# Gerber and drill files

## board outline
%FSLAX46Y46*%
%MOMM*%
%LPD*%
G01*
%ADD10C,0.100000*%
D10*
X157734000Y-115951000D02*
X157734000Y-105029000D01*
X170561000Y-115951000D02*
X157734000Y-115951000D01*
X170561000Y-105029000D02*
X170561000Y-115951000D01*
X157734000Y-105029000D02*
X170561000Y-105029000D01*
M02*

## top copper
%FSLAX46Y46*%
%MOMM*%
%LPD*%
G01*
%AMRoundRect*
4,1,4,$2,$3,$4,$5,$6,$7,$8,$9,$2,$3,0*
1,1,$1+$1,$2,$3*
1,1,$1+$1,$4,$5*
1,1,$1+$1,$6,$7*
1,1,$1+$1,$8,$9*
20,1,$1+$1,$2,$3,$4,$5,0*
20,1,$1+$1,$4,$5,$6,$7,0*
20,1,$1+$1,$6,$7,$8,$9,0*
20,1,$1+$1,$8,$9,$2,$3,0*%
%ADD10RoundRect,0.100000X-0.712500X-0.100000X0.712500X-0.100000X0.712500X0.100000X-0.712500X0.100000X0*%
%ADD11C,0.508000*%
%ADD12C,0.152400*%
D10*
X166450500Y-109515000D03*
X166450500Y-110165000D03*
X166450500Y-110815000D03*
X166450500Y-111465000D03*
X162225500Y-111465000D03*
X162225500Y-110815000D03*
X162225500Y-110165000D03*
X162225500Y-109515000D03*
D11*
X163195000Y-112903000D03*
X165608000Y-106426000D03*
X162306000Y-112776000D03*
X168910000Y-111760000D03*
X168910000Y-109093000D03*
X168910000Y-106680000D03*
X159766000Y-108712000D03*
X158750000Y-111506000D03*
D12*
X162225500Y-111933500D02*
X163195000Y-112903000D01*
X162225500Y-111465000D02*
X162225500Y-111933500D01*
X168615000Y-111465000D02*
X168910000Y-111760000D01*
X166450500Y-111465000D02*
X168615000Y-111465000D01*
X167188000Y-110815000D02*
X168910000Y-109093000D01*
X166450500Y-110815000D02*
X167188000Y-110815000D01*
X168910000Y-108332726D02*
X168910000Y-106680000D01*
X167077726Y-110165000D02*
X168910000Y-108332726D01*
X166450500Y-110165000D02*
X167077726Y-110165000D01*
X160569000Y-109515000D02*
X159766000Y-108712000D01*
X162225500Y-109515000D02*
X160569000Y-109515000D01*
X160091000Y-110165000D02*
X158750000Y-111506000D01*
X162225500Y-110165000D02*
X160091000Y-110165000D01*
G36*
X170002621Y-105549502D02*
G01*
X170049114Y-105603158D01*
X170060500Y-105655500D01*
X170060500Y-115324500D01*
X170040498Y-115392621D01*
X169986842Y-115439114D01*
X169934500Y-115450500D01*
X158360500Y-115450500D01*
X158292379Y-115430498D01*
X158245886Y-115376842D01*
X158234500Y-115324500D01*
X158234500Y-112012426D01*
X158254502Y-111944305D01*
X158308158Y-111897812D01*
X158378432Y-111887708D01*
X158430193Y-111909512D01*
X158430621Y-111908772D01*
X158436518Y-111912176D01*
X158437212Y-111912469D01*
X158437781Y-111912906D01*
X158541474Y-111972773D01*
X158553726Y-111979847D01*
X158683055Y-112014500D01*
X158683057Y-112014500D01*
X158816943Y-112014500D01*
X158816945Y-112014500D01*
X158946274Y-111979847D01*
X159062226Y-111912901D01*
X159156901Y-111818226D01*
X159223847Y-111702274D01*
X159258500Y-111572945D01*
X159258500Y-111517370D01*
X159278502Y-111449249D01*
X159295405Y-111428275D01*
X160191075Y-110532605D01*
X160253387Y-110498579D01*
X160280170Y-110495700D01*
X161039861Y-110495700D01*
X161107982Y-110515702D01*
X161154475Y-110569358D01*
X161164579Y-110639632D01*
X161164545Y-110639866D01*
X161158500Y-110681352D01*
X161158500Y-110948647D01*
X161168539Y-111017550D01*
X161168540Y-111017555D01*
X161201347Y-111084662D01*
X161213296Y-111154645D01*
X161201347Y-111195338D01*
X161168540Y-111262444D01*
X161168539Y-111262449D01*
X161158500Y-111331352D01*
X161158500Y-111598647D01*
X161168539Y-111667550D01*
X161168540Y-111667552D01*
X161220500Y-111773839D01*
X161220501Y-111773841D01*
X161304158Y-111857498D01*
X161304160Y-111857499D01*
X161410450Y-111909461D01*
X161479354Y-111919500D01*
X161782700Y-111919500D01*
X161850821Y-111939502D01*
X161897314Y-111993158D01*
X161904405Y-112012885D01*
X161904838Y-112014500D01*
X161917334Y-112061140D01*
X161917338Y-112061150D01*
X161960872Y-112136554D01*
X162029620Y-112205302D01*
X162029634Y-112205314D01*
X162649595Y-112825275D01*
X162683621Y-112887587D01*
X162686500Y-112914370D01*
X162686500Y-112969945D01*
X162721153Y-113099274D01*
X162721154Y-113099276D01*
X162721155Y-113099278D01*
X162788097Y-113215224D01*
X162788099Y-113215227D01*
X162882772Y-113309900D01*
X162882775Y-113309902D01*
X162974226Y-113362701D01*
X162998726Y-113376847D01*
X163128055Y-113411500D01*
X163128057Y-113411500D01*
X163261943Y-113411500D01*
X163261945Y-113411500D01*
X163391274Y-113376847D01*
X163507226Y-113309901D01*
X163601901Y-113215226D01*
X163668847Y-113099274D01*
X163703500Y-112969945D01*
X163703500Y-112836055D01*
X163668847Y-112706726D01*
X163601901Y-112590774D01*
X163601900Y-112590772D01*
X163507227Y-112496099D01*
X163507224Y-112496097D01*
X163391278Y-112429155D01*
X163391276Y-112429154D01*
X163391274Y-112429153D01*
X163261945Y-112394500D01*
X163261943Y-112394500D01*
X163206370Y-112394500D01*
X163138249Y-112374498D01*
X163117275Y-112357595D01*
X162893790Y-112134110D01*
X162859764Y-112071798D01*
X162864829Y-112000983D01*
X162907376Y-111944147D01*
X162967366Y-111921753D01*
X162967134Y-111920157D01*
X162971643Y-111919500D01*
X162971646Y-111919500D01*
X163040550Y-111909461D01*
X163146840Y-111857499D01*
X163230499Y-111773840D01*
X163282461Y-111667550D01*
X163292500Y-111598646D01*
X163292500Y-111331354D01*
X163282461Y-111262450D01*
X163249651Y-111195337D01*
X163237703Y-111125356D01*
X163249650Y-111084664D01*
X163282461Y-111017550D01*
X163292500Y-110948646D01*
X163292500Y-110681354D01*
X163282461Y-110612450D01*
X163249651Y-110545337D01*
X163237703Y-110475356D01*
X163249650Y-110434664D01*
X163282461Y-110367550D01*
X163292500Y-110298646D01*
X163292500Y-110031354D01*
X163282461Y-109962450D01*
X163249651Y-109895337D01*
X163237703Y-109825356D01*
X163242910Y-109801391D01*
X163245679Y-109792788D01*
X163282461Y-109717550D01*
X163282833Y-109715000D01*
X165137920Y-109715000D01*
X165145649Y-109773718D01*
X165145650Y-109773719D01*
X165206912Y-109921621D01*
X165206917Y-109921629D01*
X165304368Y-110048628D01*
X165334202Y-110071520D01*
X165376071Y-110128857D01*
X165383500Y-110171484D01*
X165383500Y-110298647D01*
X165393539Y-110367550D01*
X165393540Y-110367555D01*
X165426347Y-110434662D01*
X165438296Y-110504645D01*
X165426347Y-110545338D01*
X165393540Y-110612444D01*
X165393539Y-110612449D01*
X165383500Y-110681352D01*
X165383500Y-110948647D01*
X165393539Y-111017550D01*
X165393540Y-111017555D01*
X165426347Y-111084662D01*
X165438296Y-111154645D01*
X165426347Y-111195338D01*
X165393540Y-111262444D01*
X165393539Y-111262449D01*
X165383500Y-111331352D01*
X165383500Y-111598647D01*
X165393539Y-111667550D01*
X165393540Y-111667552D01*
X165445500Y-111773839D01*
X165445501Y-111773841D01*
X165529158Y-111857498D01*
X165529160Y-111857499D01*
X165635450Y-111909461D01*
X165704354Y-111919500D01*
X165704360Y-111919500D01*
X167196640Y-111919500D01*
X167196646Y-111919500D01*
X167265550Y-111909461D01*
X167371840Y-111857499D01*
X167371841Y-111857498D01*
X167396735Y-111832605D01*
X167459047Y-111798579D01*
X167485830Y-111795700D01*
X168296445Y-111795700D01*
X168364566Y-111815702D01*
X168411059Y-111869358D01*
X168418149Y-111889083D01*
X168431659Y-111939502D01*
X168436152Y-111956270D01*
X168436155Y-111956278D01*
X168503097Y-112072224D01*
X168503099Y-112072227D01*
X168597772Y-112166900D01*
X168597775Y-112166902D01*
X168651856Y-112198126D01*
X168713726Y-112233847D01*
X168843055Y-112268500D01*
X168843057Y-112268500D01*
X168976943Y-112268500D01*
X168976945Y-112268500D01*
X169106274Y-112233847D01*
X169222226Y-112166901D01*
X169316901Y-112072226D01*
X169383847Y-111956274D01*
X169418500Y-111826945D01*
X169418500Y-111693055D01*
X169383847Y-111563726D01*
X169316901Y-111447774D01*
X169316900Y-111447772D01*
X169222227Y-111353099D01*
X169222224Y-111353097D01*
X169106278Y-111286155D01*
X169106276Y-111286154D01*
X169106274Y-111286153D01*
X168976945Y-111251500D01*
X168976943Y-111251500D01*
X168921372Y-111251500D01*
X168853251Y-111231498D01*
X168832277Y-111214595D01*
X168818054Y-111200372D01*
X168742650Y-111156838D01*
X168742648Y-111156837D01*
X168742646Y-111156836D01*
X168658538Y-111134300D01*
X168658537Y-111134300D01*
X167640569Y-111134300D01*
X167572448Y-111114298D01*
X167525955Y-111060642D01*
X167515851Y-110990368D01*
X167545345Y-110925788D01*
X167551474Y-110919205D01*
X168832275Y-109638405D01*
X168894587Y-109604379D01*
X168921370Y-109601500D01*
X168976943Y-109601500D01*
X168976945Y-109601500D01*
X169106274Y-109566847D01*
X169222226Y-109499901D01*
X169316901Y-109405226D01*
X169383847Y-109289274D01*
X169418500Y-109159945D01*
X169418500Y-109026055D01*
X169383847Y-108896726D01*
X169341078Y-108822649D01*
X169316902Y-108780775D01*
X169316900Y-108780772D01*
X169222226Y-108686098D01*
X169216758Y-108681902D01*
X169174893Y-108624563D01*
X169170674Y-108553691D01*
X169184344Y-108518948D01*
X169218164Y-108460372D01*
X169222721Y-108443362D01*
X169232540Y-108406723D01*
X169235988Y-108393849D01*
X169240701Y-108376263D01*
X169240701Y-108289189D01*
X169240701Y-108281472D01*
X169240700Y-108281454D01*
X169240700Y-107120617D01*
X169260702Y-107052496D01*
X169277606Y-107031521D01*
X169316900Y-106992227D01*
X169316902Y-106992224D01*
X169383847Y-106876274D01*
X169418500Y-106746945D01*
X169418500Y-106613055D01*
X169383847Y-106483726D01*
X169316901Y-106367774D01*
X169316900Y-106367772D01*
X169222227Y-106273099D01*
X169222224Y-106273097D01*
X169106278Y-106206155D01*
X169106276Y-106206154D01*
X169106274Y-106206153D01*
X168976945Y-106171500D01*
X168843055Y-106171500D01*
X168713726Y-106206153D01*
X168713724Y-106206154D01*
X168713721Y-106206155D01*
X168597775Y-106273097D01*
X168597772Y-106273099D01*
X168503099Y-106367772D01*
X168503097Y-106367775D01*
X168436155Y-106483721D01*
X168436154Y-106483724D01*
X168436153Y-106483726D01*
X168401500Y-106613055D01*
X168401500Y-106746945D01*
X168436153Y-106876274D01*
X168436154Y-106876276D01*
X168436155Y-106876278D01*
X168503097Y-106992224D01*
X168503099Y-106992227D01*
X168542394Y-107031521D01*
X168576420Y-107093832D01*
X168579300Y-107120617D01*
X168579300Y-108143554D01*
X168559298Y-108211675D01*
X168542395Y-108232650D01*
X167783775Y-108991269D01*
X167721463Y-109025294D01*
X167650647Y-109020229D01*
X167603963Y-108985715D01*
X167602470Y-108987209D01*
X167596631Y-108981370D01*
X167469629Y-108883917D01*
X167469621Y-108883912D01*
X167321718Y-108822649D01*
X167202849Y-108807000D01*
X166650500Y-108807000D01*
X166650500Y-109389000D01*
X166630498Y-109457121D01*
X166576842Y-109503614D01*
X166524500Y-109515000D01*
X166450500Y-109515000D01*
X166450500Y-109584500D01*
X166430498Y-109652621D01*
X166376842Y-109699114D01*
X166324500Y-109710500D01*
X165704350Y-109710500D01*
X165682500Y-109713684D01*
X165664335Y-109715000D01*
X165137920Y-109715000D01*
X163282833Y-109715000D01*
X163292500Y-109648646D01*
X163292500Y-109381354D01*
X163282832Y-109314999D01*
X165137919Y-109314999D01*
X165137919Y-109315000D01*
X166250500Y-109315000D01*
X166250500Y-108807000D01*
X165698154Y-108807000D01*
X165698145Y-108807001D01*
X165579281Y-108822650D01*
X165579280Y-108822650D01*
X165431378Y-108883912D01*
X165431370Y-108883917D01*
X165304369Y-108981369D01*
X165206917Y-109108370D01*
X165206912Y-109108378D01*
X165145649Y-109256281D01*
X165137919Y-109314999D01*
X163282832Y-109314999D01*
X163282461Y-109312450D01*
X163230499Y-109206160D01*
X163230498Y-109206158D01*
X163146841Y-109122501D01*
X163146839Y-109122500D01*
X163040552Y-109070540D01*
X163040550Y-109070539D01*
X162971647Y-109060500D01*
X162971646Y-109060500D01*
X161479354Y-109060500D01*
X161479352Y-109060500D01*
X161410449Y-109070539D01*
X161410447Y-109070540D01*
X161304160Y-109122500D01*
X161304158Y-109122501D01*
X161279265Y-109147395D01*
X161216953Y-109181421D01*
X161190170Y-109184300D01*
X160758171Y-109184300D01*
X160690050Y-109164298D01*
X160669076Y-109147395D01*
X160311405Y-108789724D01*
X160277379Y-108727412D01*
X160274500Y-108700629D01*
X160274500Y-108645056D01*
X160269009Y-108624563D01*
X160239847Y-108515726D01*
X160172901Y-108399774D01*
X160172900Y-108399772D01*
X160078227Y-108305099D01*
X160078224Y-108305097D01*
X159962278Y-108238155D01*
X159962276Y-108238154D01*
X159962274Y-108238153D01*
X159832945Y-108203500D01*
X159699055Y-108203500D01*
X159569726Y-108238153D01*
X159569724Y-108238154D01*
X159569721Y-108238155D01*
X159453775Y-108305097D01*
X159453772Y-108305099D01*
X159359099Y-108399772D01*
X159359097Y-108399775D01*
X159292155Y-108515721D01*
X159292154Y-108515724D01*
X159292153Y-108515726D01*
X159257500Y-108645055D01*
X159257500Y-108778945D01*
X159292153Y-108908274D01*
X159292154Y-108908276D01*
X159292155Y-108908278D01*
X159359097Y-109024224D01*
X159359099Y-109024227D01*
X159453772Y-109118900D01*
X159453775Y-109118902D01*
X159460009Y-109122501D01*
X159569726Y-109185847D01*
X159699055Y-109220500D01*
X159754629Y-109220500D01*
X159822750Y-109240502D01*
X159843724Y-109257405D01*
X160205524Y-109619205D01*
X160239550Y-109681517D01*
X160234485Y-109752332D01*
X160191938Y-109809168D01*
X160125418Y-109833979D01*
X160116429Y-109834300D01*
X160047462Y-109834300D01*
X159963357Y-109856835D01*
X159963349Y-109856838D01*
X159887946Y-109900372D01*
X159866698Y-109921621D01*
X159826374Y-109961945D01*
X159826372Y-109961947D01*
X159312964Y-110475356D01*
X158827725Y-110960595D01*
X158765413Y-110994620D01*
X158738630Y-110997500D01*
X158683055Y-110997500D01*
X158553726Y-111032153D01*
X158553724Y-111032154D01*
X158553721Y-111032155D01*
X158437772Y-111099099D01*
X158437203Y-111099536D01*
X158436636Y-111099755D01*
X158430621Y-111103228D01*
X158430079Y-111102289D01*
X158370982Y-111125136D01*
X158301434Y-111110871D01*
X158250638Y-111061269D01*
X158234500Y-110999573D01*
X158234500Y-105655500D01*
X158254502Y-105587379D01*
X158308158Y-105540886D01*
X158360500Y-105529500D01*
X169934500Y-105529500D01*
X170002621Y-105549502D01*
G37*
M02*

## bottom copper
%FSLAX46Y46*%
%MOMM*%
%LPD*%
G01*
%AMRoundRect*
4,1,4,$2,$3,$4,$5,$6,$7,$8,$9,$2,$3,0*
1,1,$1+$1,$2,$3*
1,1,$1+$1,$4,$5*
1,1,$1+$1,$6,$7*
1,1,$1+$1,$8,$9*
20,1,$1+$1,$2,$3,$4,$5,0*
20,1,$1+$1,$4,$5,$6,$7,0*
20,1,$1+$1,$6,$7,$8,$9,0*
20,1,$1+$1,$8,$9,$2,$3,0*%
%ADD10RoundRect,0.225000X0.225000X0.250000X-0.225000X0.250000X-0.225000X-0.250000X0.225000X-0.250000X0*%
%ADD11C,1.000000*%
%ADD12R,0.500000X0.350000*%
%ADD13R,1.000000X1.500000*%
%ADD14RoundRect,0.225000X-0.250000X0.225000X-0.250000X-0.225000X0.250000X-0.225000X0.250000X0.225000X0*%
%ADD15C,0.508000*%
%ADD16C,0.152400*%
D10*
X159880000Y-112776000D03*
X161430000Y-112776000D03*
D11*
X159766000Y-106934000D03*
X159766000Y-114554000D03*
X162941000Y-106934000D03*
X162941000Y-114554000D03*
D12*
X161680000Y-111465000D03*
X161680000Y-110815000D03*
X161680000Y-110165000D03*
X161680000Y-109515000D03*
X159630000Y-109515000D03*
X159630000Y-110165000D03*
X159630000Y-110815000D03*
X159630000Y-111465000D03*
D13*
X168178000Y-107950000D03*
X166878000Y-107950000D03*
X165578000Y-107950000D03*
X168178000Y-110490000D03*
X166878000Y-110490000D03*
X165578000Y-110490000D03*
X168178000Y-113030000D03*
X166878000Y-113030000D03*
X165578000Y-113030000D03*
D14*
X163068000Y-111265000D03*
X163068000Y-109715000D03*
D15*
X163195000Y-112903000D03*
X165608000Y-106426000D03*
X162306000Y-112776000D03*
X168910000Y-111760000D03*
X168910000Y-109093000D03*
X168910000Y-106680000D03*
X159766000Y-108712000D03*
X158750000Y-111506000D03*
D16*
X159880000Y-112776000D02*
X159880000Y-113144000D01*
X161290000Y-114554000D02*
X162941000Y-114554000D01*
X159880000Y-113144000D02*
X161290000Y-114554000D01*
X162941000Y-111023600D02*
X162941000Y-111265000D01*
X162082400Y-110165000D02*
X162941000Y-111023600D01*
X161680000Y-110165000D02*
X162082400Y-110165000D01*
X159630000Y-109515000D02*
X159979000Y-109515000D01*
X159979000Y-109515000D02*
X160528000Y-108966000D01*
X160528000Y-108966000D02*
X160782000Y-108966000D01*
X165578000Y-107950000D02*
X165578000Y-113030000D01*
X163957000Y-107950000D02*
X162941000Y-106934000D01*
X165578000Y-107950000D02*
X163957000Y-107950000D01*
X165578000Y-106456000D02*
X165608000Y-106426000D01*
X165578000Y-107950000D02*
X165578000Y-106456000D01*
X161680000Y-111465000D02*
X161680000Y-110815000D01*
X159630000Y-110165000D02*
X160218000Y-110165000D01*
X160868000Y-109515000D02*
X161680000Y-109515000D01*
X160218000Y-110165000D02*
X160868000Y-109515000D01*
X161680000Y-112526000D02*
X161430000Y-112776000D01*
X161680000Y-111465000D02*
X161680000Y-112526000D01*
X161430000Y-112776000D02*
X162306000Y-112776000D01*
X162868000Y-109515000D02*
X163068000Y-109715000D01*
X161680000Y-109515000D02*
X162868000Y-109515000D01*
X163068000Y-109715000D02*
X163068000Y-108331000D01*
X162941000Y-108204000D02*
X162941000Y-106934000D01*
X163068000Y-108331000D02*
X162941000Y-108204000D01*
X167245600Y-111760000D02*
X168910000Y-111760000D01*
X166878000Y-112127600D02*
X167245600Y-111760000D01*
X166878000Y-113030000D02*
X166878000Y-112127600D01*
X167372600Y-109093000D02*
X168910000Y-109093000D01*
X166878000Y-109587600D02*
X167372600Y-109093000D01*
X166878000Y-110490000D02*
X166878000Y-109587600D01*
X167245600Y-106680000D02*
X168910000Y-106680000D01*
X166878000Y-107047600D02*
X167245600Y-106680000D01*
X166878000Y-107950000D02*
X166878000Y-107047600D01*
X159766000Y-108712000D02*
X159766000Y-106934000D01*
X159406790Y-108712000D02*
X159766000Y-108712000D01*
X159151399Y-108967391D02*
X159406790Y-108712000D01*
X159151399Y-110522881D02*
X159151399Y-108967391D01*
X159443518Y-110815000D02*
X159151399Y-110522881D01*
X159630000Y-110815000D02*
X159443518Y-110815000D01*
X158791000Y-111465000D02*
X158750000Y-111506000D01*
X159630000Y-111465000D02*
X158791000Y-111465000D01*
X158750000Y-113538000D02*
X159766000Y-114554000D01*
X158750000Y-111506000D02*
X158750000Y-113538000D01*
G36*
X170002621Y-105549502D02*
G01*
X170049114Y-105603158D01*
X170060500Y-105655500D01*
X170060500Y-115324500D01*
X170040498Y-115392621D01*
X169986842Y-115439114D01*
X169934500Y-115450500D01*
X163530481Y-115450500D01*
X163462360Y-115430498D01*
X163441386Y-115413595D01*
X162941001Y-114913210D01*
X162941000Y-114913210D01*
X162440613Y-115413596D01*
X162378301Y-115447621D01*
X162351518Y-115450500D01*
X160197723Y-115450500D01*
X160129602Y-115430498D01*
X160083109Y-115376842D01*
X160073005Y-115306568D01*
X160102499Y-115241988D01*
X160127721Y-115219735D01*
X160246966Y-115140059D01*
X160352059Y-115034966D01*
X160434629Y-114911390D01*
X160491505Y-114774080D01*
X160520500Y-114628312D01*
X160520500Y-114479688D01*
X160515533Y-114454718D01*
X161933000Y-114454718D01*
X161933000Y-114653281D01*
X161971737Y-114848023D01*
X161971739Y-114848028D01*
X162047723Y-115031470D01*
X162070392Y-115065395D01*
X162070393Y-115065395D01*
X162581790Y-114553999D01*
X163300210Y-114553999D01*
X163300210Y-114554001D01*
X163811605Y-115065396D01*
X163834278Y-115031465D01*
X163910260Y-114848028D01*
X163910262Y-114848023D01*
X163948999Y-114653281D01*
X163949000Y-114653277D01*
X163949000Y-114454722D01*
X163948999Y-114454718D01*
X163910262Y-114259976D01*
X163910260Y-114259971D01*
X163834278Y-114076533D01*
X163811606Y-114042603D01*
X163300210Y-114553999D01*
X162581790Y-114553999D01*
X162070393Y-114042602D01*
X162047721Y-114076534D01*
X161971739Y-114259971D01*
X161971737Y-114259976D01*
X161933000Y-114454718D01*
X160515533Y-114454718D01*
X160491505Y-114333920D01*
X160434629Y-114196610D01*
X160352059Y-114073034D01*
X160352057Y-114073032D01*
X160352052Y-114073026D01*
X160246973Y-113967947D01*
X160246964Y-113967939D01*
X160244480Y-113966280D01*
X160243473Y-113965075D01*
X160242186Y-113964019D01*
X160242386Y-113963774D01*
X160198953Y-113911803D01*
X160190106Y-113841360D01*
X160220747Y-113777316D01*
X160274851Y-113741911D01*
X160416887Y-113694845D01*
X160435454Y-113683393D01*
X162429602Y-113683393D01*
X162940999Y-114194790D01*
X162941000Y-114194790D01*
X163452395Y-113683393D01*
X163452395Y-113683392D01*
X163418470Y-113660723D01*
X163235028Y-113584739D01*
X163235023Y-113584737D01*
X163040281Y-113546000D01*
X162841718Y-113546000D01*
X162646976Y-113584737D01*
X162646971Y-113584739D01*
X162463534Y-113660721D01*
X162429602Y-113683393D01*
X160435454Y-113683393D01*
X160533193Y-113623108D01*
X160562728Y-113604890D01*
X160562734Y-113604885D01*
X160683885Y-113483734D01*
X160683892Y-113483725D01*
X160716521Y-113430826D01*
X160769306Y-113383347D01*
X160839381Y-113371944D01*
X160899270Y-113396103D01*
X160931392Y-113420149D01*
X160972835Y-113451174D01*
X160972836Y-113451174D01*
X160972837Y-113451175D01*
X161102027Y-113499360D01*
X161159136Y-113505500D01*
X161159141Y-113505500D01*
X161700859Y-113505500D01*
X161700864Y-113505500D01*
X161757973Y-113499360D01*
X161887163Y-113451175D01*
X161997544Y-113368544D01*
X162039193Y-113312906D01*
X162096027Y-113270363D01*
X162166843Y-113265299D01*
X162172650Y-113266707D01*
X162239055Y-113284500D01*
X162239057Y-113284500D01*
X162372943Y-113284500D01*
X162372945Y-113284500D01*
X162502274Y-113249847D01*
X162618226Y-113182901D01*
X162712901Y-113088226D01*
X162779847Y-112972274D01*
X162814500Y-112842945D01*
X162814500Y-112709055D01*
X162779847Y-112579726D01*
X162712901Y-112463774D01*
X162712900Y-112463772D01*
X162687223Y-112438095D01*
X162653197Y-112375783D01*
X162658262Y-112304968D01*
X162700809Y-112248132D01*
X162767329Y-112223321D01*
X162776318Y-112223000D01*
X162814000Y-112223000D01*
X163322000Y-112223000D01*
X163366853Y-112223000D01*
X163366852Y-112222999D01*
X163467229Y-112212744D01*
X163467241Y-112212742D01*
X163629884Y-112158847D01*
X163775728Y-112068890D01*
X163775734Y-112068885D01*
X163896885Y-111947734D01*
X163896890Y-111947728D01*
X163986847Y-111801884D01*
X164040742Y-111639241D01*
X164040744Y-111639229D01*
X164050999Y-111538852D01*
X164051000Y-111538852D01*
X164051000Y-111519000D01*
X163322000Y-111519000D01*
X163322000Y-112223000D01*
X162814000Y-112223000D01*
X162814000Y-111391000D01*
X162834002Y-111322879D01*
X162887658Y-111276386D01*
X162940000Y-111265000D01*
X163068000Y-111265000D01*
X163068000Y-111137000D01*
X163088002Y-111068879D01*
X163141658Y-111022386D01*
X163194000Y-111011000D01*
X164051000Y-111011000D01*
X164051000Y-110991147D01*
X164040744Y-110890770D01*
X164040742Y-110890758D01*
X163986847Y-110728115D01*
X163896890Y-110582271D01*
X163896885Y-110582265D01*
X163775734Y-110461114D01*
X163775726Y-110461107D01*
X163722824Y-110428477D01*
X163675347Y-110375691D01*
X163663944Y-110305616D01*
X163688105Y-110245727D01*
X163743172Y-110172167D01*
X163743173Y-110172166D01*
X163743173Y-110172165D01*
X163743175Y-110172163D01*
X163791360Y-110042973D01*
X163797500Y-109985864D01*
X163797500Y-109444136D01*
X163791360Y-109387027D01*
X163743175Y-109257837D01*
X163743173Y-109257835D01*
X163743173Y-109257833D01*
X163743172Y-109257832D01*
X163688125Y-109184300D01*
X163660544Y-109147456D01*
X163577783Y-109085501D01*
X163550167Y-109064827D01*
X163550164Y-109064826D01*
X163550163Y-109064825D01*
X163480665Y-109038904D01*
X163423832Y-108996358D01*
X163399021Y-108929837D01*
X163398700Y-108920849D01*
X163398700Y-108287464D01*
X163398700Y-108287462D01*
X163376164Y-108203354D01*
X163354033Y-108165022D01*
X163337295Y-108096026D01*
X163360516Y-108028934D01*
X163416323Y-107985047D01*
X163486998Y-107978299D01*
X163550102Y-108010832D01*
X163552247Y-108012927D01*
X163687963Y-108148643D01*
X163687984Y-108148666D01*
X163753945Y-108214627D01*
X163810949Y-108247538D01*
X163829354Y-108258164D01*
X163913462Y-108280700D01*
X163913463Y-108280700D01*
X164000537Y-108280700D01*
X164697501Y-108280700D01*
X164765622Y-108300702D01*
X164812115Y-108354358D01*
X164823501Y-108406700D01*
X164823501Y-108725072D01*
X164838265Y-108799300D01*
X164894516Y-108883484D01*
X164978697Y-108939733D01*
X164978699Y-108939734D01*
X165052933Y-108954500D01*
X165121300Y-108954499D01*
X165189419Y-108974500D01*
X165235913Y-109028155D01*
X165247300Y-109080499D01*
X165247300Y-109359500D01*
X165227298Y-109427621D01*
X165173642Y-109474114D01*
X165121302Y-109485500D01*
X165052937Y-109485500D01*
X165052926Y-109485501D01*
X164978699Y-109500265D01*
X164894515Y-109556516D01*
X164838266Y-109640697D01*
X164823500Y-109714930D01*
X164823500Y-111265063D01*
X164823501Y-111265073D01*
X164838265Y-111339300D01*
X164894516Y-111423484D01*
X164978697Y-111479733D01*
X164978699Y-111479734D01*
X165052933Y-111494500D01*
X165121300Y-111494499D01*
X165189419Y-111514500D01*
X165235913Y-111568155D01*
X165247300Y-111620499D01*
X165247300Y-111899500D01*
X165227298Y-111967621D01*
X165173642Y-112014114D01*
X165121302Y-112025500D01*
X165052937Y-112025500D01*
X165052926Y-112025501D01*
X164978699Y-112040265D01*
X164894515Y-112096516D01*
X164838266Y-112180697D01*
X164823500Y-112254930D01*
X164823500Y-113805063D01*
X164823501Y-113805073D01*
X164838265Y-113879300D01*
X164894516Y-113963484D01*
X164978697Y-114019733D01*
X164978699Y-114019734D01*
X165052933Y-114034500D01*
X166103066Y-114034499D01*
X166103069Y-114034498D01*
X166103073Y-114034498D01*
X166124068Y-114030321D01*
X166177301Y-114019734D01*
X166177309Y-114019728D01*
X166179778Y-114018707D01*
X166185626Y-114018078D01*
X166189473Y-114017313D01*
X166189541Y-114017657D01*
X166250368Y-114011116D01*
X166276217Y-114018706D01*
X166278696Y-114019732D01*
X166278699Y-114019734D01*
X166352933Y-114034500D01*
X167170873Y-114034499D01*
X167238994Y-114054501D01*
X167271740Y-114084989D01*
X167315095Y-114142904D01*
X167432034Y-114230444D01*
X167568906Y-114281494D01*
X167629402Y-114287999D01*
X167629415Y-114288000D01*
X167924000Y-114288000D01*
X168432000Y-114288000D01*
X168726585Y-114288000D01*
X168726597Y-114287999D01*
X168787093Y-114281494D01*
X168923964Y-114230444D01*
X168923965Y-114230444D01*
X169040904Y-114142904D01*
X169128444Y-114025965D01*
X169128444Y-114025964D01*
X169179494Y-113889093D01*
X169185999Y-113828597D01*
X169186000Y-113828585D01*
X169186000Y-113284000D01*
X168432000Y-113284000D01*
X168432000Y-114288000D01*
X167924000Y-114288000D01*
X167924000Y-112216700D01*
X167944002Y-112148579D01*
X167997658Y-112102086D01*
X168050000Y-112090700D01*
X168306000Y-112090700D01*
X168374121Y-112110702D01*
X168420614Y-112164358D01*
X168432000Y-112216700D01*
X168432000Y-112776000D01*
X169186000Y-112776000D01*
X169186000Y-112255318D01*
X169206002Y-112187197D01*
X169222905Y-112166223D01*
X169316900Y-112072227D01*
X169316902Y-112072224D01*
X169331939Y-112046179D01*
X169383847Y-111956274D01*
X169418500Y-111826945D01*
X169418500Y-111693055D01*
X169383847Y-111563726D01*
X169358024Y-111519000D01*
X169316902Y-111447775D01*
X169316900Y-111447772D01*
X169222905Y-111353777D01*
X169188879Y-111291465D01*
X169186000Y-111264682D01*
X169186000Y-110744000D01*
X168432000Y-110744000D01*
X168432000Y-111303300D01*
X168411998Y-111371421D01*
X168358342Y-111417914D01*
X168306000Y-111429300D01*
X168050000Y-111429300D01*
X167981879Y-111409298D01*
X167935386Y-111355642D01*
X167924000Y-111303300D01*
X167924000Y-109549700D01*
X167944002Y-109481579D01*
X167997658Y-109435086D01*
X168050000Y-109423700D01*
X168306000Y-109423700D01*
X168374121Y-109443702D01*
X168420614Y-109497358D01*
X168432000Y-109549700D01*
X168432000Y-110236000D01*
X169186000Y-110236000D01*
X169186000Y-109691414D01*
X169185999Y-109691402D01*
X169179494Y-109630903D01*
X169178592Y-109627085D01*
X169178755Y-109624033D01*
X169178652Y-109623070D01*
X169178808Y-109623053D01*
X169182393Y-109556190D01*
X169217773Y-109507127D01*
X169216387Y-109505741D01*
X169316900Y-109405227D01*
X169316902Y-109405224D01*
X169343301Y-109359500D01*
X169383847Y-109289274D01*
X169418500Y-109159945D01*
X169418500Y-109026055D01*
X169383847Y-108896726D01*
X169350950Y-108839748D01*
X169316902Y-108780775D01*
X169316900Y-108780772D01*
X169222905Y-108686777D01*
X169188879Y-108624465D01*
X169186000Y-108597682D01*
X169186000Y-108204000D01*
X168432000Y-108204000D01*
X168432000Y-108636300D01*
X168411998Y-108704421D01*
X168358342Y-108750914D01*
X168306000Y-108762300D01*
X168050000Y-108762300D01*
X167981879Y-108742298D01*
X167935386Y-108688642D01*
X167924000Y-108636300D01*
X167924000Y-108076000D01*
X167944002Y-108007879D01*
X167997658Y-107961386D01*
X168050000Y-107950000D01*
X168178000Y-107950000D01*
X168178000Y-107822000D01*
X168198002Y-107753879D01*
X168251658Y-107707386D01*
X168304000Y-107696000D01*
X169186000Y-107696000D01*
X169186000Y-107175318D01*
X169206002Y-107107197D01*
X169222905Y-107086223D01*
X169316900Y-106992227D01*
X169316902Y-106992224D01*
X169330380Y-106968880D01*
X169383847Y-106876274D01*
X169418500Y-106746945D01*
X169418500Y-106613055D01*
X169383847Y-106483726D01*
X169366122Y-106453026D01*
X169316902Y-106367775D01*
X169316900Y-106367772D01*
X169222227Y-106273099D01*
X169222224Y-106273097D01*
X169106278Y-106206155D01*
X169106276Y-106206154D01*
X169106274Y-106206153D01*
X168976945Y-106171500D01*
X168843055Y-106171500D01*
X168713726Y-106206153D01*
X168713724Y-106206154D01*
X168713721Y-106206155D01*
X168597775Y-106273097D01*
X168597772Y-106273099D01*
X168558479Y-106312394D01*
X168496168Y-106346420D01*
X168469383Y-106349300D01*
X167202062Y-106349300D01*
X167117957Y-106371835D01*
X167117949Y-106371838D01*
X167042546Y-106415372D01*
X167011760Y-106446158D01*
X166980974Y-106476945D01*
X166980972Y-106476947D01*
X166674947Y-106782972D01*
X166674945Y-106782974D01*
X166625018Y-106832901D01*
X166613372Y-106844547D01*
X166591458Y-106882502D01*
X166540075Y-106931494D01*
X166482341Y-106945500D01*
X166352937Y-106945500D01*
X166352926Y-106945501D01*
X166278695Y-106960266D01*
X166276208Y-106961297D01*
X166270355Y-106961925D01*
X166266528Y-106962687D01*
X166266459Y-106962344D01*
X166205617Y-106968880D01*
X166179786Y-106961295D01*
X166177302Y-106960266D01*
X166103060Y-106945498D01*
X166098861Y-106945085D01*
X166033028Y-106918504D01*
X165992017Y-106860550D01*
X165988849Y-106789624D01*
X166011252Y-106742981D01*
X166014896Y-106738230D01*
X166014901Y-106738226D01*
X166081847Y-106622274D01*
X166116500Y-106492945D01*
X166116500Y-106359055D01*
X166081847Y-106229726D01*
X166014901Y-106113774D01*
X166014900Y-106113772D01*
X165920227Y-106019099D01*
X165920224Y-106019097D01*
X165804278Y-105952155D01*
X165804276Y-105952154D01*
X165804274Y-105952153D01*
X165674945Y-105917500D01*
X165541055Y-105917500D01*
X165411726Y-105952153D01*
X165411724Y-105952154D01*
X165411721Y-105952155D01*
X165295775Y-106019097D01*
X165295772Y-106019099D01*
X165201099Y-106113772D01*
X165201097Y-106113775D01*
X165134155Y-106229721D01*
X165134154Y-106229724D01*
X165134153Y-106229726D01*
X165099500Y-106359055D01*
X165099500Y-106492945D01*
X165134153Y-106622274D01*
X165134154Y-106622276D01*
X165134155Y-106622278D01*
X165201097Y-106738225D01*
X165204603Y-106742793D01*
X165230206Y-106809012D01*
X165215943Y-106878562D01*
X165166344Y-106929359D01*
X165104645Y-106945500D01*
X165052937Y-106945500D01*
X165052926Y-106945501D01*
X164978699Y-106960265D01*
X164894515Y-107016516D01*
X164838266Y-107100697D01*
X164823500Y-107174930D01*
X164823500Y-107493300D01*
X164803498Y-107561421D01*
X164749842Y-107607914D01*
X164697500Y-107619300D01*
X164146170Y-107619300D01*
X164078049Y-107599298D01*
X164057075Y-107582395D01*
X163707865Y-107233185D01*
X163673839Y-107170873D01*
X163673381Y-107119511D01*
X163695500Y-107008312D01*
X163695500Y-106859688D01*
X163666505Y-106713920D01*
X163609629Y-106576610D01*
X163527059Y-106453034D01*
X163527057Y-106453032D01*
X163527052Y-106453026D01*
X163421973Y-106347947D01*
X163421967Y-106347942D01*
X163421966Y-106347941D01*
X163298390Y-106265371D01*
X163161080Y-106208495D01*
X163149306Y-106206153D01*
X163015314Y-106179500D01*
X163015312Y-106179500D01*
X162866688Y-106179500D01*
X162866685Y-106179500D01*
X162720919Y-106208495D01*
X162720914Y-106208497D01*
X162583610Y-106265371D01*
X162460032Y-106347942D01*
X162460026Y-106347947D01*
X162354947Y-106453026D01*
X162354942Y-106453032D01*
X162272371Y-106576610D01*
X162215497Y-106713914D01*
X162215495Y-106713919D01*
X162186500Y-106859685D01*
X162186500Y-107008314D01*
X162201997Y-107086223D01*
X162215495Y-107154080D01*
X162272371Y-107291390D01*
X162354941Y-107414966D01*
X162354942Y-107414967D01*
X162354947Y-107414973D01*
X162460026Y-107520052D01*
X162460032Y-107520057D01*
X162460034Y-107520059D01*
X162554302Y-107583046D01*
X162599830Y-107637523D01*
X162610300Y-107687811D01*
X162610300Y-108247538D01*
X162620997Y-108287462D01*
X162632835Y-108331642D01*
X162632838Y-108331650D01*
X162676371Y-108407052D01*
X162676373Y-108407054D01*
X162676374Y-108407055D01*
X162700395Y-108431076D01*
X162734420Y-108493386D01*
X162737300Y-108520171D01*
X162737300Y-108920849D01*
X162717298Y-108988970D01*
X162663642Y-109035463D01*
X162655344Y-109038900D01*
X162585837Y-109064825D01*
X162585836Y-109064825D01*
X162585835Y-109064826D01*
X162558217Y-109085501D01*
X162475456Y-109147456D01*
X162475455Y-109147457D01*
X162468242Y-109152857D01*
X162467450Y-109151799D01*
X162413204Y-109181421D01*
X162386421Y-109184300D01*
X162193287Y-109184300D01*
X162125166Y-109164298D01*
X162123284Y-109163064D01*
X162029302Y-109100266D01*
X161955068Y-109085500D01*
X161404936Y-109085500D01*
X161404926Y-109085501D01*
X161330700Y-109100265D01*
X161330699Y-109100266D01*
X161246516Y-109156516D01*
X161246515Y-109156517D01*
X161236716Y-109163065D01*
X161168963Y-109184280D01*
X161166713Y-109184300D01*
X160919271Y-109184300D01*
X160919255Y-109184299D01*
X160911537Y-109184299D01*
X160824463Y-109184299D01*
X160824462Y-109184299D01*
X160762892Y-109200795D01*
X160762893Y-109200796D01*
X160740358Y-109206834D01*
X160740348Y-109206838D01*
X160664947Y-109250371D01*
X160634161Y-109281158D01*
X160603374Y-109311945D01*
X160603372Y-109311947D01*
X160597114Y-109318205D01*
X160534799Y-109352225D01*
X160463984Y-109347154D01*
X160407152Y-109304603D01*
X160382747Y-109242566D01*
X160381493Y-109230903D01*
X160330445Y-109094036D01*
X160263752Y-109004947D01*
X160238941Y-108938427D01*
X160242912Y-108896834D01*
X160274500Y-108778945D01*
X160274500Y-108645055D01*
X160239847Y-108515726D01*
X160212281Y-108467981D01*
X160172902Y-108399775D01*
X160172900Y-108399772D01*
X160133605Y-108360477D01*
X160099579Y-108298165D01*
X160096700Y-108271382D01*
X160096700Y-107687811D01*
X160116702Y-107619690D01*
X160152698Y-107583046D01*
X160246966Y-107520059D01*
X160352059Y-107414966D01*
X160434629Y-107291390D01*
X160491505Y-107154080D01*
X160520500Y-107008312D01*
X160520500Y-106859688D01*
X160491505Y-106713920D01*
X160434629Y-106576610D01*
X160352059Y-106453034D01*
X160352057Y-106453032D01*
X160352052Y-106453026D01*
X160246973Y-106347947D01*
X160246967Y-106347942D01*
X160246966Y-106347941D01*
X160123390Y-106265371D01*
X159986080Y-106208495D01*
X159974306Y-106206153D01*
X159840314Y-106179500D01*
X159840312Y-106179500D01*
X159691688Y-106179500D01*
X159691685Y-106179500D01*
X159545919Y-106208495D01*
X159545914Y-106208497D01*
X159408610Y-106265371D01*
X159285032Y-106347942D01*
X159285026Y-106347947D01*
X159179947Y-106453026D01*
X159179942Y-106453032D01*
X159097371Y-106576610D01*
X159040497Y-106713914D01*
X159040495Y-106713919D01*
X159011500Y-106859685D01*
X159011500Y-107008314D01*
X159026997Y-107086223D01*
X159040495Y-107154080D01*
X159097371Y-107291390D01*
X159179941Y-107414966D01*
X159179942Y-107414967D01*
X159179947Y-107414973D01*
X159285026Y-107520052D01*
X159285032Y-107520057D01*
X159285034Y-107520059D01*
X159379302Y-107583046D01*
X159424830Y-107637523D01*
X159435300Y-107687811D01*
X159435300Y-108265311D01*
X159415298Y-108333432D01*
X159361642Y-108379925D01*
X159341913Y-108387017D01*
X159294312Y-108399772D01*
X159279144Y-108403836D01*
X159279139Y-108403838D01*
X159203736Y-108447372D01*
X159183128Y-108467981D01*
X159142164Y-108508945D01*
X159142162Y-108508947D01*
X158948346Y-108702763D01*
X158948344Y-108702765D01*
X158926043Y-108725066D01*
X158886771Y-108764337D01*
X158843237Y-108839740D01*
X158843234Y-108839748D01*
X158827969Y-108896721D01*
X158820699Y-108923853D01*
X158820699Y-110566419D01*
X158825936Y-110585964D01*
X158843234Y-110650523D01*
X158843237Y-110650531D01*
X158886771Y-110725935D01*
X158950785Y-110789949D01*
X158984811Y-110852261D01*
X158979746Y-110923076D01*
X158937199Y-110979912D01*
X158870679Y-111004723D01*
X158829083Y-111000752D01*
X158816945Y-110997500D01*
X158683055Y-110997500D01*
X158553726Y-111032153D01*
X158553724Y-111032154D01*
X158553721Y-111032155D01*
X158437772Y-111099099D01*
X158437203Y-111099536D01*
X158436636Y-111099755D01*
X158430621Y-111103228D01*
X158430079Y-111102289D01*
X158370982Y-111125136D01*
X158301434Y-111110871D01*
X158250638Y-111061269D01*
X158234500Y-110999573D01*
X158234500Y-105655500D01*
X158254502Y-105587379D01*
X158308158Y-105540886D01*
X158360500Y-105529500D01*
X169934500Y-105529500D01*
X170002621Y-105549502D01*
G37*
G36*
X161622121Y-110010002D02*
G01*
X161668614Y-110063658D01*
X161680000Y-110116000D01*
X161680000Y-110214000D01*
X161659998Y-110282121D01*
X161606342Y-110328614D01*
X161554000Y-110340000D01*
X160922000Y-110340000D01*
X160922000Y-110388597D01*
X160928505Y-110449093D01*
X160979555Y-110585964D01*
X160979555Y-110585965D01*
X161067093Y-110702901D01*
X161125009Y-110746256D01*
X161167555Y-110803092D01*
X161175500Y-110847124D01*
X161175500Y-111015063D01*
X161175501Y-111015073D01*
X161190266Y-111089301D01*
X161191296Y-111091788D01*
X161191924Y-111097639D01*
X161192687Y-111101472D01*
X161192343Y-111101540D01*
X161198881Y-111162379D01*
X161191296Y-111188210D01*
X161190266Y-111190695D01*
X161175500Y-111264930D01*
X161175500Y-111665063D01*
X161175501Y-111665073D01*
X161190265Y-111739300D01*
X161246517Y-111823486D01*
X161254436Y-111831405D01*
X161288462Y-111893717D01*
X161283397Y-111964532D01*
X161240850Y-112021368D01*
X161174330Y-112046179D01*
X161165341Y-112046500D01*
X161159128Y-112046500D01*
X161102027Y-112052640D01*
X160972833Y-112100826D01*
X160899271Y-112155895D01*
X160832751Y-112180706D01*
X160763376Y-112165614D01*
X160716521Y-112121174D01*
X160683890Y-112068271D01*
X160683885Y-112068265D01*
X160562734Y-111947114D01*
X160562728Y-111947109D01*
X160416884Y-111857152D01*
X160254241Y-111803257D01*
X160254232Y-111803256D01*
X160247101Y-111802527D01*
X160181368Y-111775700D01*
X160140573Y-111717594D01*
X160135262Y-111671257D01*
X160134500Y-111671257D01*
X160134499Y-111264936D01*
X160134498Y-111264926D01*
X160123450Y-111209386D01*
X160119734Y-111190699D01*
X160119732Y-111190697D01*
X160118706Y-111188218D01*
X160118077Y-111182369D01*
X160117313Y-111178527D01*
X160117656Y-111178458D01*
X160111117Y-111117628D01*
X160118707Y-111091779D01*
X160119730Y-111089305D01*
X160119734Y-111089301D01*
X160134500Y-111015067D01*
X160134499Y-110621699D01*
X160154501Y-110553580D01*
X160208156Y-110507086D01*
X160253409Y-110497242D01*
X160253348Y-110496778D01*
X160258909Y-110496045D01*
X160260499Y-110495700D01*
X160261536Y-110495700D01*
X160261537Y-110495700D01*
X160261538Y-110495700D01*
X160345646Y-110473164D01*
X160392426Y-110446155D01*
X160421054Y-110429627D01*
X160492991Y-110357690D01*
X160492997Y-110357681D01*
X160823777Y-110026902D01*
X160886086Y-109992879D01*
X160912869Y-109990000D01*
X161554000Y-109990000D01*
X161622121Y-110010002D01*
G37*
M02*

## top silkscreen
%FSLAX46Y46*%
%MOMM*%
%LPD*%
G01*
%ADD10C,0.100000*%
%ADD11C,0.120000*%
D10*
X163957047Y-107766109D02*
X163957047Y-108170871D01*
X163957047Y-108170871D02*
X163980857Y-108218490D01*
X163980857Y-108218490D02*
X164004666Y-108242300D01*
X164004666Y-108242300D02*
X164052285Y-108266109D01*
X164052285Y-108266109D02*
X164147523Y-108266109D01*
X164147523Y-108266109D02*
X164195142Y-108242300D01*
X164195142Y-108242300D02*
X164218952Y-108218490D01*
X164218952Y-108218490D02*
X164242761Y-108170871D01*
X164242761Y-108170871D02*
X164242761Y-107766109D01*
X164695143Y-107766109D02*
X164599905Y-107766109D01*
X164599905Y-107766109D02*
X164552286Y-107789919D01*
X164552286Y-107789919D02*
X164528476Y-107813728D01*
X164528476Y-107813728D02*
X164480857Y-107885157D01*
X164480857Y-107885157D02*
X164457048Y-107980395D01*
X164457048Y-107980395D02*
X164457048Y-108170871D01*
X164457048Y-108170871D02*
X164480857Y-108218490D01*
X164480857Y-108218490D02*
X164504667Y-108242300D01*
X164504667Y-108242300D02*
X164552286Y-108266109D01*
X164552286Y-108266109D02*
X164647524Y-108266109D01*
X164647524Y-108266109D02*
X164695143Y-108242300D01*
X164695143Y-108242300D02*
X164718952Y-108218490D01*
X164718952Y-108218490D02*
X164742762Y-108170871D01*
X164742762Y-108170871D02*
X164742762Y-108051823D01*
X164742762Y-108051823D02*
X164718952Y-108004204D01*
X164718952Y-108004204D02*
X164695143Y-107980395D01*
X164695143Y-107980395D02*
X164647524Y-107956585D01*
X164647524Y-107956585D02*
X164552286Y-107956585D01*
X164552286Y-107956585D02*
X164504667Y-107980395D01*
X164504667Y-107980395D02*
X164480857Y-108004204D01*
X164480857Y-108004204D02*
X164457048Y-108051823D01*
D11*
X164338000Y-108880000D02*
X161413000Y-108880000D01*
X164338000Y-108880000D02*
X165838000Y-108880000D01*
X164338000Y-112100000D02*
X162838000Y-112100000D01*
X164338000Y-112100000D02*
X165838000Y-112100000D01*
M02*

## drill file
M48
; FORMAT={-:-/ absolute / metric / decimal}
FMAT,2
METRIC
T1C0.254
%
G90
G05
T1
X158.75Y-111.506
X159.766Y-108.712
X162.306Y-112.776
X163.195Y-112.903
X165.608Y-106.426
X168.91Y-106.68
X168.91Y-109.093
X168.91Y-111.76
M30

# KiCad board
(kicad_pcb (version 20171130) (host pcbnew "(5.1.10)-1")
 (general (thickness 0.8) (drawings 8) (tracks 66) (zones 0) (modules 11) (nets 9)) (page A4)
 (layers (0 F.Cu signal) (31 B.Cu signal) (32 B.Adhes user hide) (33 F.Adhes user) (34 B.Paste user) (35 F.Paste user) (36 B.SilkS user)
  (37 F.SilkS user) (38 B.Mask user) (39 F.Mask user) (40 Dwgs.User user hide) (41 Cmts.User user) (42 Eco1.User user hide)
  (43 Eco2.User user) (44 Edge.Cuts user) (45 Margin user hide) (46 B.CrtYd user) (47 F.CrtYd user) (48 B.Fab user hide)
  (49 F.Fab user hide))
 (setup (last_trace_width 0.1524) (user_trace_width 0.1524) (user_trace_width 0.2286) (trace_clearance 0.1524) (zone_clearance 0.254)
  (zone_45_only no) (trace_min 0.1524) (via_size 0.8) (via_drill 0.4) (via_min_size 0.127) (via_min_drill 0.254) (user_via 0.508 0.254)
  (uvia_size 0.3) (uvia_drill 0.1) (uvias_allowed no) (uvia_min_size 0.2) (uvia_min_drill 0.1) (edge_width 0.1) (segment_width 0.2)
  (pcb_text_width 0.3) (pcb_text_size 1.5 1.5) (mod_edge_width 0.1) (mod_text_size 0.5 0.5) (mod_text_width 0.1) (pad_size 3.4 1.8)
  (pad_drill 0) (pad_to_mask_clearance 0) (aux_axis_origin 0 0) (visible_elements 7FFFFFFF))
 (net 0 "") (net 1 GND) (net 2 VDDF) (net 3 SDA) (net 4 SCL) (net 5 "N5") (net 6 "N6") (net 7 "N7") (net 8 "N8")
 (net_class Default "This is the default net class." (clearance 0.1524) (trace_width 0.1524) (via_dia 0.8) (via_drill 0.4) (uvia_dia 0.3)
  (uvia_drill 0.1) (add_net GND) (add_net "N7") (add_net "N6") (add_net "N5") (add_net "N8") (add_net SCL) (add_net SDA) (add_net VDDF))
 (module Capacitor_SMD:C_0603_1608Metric (layer B.Cu) (at 160.655 112.776 180)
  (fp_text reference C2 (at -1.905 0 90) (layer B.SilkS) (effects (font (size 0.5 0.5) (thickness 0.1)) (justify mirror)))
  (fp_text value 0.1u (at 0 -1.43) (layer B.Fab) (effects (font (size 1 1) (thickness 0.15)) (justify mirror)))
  (pad 2 smd roundrect (at 0.775 0 180) (size 0.9 0.95) (layers B.Cu B.Paste B.Mask) (roundrect_rratio 0.25) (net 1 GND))
  (pad 1 smd roundrect (at -0.775 0 180) (size 0.9 0.95) (layers B.Cu B.Paste B.Mask) (roundrect_rratio 0.25) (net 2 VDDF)))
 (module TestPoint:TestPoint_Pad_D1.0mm (layer B.Cu) (at 159.766 106.934)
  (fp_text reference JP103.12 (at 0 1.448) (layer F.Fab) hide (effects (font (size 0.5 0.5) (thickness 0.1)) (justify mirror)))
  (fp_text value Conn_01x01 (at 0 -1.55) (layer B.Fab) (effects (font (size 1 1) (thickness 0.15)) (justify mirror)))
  (pad 1 smd circle (at 0 0) (size 1 1) (layers B.Cu B.Mask) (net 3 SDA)))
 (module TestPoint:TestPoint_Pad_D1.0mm (layer B.Cu) (at 159.766 114.554)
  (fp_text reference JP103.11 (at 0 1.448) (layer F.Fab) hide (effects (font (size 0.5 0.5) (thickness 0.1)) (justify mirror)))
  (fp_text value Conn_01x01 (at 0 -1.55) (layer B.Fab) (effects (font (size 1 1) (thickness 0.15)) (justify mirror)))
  (pad 1 smd circle (at 0 0) (size 1 1) (layers B.Cu B.Mask) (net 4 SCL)))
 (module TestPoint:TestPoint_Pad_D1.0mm (layer B.Cu) (at 162.941 106.934)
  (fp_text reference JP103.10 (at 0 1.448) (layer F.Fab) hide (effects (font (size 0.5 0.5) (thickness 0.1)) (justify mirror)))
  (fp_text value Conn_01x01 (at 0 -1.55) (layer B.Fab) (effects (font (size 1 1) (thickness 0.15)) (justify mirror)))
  (pad 1 smd circle (at 0 0) (size 1 1) (layers B.Cu B.Mask) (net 2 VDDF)))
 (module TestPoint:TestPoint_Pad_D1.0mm (layer B.Cu) (at 162.941 114.554 90)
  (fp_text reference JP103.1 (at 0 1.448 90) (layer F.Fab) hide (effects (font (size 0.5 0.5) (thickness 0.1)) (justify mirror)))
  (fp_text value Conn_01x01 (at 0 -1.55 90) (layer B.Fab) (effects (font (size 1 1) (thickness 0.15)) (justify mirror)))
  (pad 1 smd circle (at 0 0 90) (size 1 1) (layers B.Cu B.Mask) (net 1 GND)))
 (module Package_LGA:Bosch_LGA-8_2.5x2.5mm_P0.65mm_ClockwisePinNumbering (layer B.Cu) (at 160.655 110.49 270)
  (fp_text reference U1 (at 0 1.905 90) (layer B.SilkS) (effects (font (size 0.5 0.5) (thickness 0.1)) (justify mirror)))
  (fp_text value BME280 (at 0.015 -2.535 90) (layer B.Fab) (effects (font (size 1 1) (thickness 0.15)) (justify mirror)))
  (pad 5 smd rect (at 0.975 -1.025 180) (size 0.5 0.35) (layers B.Cu B.Paste B.Mask) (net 2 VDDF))
  (pad 6 smd rect (at 0.325 -1.025 180) (size 0.5 0.35) (layers B.Cu B.Paste B.Mask) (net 2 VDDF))
  (pad 7 smd rect (at -0.325 -1.025 180) (size 0.5 0.35) (layers B.Cu B.Paste B.Mask) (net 1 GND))
  (pad 8 smd rect (at -0.975 -1.025 180) (size 0.5 0.35) (layers B.Cu B.Paste B.Mask) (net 2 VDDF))
  (pad 1 smd rect (at -0.975 1.025 180) (size 0.5 0.35) (layers B.Cu B.Paste B.Mask) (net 1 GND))
  (pad 2 smd rect (at -0.325 1.025 180) (size 0.5 0.35) (layers B.Cu B.Paste B.Mask) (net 2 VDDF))
  (pad 3 smd rect (at 0.325 1.025 180) (size 0.5 0.35) (layers B.Cu B.Paste B.Mask) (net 3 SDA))
  (pad 4 smd rect (at 0.975 1.025 180) (size 0.5 0.35) (layers B.Cu B.Paste B.Mask) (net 4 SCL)))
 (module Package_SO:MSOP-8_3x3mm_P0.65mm (layer F.Cu) (at 164.338 110.49)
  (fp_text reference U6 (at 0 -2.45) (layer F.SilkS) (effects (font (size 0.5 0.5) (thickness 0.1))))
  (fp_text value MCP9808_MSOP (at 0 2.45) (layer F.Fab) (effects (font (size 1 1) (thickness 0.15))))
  (fp_line (start 0 -1.61) (end -2.925 -1.61) (layer F.SilkS) (width 0.12))
  (fp_line (start 0 -1.61) (end 1.5 -1.61) (layer F.SilkS) (width 0.12))
  (fp_line (start 0 1.61) (end -1.5 1.61) (layer F.SilkS) (width 0.12))
  (fp_line (start 0 1.61) (end 1.5 1.61) (layer F.SilkS) (width 0.12))
  (pad 8 smd roundrect (at 2.1125 -0.975) (size 1.625 0.4) (layers F.Cu F.Paste F.Mask) (roundrect_rratio 0.25) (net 2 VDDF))
  (pad 7 smd roundrect (at 2.1125 -0.325) (size 1.625 0.4) (layers F.Cu F.Paste F.Mask) (roundrect_rratio 0.25) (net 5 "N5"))
  (pad 6 smd roundrect (at 2.1125 0.325) (size 1.625 0.4) (layers F.Cu F.Paste F.Mask) (roundrect_rratio 0.25) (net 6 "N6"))
  (pad 5 smd roundrect (at 2.1125 0.975) (size 1.625 0.4) (layers F.Cu F.Paste F.Mask) (roundrect_rratio 0.25) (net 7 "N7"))
  (pad 4 smd roundrect (at -2.1125 0.975) (size 1.625 0.4) (layers F.Cu F.Paste F.Mask) (roundrect_rratio 0.25) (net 1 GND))
  (pad 3 smd roundrect (at -2.1125 0.325) (size 1.625 0.4) (layers F.Cu F.Paste F.Mask) (roundrect_rratio 0.25) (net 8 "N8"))
  (pad 2 smd roundrect (at -2.1125 -0.325) (size 1.625 0.4) (layers F.Cu F.Paste F.Mask) (roundrect_rratio 0.25) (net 4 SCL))
  (pad 1 smd roundrect (at -2.1125 -0.975) (size 1.625 0.4) (layers F.Cu F.Paste F.Mask) (roundrect_rratio 0.25) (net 3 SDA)))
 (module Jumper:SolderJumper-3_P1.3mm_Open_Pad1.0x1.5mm (layer B.Cu) (at 166.878 107.95 180)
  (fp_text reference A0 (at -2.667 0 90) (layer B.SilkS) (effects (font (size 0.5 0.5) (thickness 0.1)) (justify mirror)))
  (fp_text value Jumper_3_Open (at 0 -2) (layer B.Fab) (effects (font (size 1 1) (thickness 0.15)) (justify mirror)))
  (pad 1 smd rect (at -1.3 0 180) (size 1 1.5) (layers B.Cu B.Mask) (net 1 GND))
  (pad 2 smd rect (at 0 0 180) (size 1 1.5) (layers B.Cu B.Mask) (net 5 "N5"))
  (pad 3 smd rect (at 1.3 0 180) (size 1 1.5) (layers B.Cu B.Mask) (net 2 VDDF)))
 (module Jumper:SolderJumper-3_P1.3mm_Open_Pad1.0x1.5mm (layer B.Cu) (at 166.878 110.49 180)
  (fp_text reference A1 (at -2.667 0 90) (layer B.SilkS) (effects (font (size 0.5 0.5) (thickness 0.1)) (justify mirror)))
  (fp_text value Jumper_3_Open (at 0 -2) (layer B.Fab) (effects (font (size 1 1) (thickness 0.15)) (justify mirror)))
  (pad 1 smd rect (at -1.3 0 180) (size 1 1.5) (layers B.Cu B.Mask) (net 1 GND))
  (pad 2 smd rect (at 0 0 180) (size 1 1.5) (layers B.Cu B.Mask) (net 6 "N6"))
  (pad 3 smd rect (at 1.3 0 180) (size 1 1.5) (layers B.Cu B.Mask) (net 2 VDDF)))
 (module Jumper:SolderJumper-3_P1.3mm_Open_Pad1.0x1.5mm (layer B.Cu) (at 166.878 113.03 180)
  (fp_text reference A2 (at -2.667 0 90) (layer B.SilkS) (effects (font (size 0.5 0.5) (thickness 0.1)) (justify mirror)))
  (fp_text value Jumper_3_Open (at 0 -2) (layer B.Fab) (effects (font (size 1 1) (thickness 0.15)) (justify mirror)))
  (pad 1 smd rect (at -1.3 0 180) (size 1 1.5) (layers B.Cu B.Mask) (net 1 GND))
  (pad 2 smd rect (at 0 0 180) (size 1 1.5) (layers B.Cu B.Mask) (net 7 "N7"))
  (pad 3 smd rect (at 1.3 0 180) (size 1 1.5) (layers B.Cu B.Mask) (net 2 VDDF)))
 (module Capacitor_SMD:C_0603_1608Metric (layer B.Cu) (at 163.068 110.49 270)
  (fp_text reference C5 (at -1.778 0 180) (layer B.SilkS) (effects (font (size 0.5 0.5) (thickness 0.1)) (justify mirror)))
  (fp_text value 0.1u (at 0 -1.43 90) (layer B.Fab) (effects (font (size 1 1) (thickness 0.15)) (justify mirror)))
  (pad 2 smd roundrect (at 0.775 0 270) (size 0.9 0.95) (layers B.Cu B.Paste B.Mask) (roundrect_rratio 0.25) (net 1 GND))
  (pad 1 smd roundrect (at -0.775 0 270) (size 0.9 0.95) (layers B.Cu B.Paste B.Mask) (roundrect_rratio 0.25) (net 2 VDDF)))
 (gr_line (start 157.734 115.951) (end 157.734 105.029) (layer Edge.Cuts) (width 0.1))
 (gr_line (start 170.561 115.951) (end 157.734 115.951) (layer Edge.Cuts) (width 0.1))
 (gr_line (start 170.561 105.029) (end 170.561 115.951) (layer Edge.Cuts) (width 0.1))
 (gr_line (start 157.734 105.029) (end 170.561 105.029) (layer Edge.Cuts) (width 0.1))
 (segment (start 159.88 112.776) (end 159.88 113.144) (width 0.1524) (layer B.Cu) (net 1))
 (segment (start 161.29 114.554) (end 162.941 114.554) (width 0.1524) (layer B.Cu) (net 1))
 (segment (start 159.88 113.144) (end 161.29 114.554) (width 0.1524) (layer B.Cu) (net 1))
 (segment (start 162.941 111.0236) (end 162.941 111.265) (width 0.1524) (layer B.Cu) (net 1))
 (segment (start 162.0824 110.165) (end 162.941 111.0236) (width 0.1524) (layer B.Cu) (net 1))
 (segment (start 161.68 110.165) (end 162.0824 110.165) (width 0.1524) (layer B.Cu) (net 1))
 (segment (start 159.63 109.515) (end 159.979 109.515) (width 0.1524) (layer B.Cu) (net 1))
 (segment (start 159.979 109.515) (end 160.528 108.966) (width 0.1524) (layer B.Cu) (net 1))
 (segment (start 160.528 108.966) (end 160.782 108.966) (width 0.1524) (layer B.Cu) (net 1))
 (via (at 163.195 112.903) (size 0.508) (drill 0.254) (layers F.Cu B.Cu) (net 1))
 (segment (start 162.2255 111.9335) (end 163.195 112.903) (width 0.1524) (layer F.Cu) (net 1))
 (segment (start 162.2255 111.465) (end 162.2255 111.9335) (width 0.1524) (layer F.Cu) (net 1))
 (segment (start 165.578 107.95) (end 165.578 113.03) (width 0.1524) (layer B.Cu) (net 2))
 (segment (start 163.957 107.95) (end 162.941 106.934) (width 0.1524) (layer B.Cu) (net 2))
 (segment (start 165.578 107.95) (end 163.957 107.95) (width 0.1524) (layer B.Cu) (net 2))
 (via (at 165.608 106.426) (size 0.508) (drill 0.254) (layers F.Cu B.Cu) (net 2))
 (segment (start 165.578 106.456) (end 165.608 106.426) (width 0.1524) (layer B.Cu) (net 2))
 (segment (start 165.578 107.95) (end 165.578 106.456) (width 0.1524) (layer B.Cu) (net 2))
 (segment (start 161.68 111.465) (end 161.68 110.815) (width 0.1524) (layer B.Cu) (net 2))
 (segment (start 159.63 110.165) (end 160.218 110.165) (width 0.1524) (layer B.Cu) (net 2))
 (segment (start 160.868 109.515) (end 161.68 109.515) (width 0.1524) (layer B.Cu) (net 2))
 (segment (start 160.218 110.165) (end 160.868 109.515) (width 0.1524) (layer B.Cu) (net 2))
 (segment (start 161.68 112.526) (end 161.43 112.776) (width 0.1524) (layer B.Cu) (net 2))
 (segment (start 161.68 111.465) (end 161.68 112.526) (width 0.1524) (layer B.Cu) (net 2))
 (via (at 162.306 112.776) (size 0.508) (drill 0.254) (layers F.Cu B.Cu) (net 2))
 (segment (start 161.43 112.776) (end 162.306 112.776) (width 0.1524) (layer B.Cu) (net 2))
 (segment (start 162.868 109.515) (end 163.068 109.715) (width 0.1524) (layer B.Cu) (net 2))
 (segment (start 161.68 109.515) (end 162.868 109.515) (width 0.1524) (layer B.Cu) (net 2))
 (segment (start 163.068 109.715) (end 163.068 108.331) (width 0.1524) (layer B.Cu) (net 2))
 (segment (start 162.941 108.204) (end 162.941 106.934) (width 0.1524) (layer B.Cu) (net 2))
 (segment (start 163.068 108.331) (end 162.941 108.204) (width 0.1524) (layer B.Cu) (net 2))
 (via (at 168.91 111.76) (size 0.508) (drill 0.254) (layers F.Cu B.Cu) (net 7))
 (segment (start 167.2456 111.76) (end 168.91 111.76) (width 0.1524) (layer B.Cu) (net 7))
 (segment (start 166.878 112.1276) (end 167.2456 111.76) (width 0.1524) (layer B.Cu) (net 7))
 (segment (start 166.878 113.03) (end 166.878 112.1276) (width 0.1524) (layer B.Cu) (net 7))
 (segment (start 168.615 111.465) (end 168.91 111.76) (width 0.1524) (layer F.Cu) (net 7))
 (segment (start 166.4505 111.465) (end 168.615 111.465) (width 0.1524) (layer F.Cu) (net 7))
 (via (at 168.91 109.093) (size 0.508) (drill 0.254) (layers F.Cu B.Cu) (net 6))
 (segment (start 167.3726 109.093) (end 168.91 109.093) (width 0.1524) (layer B.Cu) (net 6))
 (segment (start 166.878 109.5876) (end 167.3726 109.093) (width 0.1524) (layer B.Cu) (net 6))
 (segment (start 166.878 110.49) (end 166.878 109.5876) (width 0.1524) (layer B.Cu) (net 6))
 (segment (start 167.188 110.815) (end 168.91 109.093) (width 0.1524) (layer F.Cu) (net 6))
 (segment (start 166.4505 110.815) (end 167.188 110.815) (width 0.1524) (layer F.Cu) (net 6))
 (via (at 168.91 106.68) (size 0.508) (drill 0.254) (layers F.Cu B.Cu) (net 5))
 (segment (start 167.2456 106.68) (end 168.91 106.68) (width 0.1524) (layer B.Cu) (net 5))
 (segment (start 166.878 107.0476) (end 167.2456 106.68) (width 0.1524) (layer B.Cu) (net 5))
 (segment (start 166.878 107.95) (end 166.878 107.0476) (width 0.1524) (layer B.Cu) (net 5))
 (segment (start 168.91 108.332726) (end 168.91 106.68) (width 0.1524) (layer F.Cu) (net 5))
 (segment (start 167.077726 110.165) (end 168.91 108.332726) (width 0.1524) (layer F.Cu) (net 5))
 (segment (start 166.4505 110.165) (end 167.077726 110.165) (width 0.1524) (layer F.Cu) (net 5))
 (via (at 159.766 108.712) (size 0.508) (drill 0.254) (layers F.Cu B.Cu) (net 3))
 (segment (start 160.569 109.515) (end 159.766 108.712) (width 0.1524) (layer F.Cu) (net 3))
 (segment (start 162.2255 109.515) (end 160.569 109.515) (width 0.1524) (layer F.Cu) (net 3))
 (segment (start 159.766 108.712) (end 159.766 106.934) (width 0.1524) (layer B.Cu) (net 3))
 (segment (start 159.40679 108.712) (end 159.766 108.712) (width 0.1524) (layer B.Cu) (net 3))
 (segment (start 159.151399 108.967391) (end 159.40679 108.712) (width 0.1524) (layer B.Cu) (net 3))
 (segment (start 159.151399 110.522881) (end 159.151399 108.967391) (width 0.1524) (layer B.Cu) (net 3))
 (segment (start 159.443518 110.815) (end 159.151399 110.522881) (width 0.1524) (layer B.Cu) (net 3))
 (segment (start 159.63 110.815) (end 159.443518 110.815) (width 0.1524) (layer B.Cu) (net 3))
 (via (at 158.75 111.506) (size 0.508) (drill 0.254) (layers F.Cu B.Cu) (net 4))
 (segment (start 160.091 110.165) (end 158.75 111.506) (width 0.1524) (layer F.Cu) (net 4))
 (segment (start 162.2255 110.165) (end 160.091 110.165) (width 0.1524) (layer F.Cu) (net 4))
 (segment (start 158.791 111.465) (end 158.75 111.506) (width 0.1524) (layer B.Cu) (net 4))
 (segment (start 159.63 111.465) (end 158.791 111.465) (width 0.1524) (layer B.Cu) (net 4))
 (segment (start 158.75 113.538) (end 159.766 114.554) (width 0.1524) (layer B.Cu) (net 4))
 (segment (start 158.75 111.506) (end 158.75 113.538) (width 0.1524) (layer B.Cu) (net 4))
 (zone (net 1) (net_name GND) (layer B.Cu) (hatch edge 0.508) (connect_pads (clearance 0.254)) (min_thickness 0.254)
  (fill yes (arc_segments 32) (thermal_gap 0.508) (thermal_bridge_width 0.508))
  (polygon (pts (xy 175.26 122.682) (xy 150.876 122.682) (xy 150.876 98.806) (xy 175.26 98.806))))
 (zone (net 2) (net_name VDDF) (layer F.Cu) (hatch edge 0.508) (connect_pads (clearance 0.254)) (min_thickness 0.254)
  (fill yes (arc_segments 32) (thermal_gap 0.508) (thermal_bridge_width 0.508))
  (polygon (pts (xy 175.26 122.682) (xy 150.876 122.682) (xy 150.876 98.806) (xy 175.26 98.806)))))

